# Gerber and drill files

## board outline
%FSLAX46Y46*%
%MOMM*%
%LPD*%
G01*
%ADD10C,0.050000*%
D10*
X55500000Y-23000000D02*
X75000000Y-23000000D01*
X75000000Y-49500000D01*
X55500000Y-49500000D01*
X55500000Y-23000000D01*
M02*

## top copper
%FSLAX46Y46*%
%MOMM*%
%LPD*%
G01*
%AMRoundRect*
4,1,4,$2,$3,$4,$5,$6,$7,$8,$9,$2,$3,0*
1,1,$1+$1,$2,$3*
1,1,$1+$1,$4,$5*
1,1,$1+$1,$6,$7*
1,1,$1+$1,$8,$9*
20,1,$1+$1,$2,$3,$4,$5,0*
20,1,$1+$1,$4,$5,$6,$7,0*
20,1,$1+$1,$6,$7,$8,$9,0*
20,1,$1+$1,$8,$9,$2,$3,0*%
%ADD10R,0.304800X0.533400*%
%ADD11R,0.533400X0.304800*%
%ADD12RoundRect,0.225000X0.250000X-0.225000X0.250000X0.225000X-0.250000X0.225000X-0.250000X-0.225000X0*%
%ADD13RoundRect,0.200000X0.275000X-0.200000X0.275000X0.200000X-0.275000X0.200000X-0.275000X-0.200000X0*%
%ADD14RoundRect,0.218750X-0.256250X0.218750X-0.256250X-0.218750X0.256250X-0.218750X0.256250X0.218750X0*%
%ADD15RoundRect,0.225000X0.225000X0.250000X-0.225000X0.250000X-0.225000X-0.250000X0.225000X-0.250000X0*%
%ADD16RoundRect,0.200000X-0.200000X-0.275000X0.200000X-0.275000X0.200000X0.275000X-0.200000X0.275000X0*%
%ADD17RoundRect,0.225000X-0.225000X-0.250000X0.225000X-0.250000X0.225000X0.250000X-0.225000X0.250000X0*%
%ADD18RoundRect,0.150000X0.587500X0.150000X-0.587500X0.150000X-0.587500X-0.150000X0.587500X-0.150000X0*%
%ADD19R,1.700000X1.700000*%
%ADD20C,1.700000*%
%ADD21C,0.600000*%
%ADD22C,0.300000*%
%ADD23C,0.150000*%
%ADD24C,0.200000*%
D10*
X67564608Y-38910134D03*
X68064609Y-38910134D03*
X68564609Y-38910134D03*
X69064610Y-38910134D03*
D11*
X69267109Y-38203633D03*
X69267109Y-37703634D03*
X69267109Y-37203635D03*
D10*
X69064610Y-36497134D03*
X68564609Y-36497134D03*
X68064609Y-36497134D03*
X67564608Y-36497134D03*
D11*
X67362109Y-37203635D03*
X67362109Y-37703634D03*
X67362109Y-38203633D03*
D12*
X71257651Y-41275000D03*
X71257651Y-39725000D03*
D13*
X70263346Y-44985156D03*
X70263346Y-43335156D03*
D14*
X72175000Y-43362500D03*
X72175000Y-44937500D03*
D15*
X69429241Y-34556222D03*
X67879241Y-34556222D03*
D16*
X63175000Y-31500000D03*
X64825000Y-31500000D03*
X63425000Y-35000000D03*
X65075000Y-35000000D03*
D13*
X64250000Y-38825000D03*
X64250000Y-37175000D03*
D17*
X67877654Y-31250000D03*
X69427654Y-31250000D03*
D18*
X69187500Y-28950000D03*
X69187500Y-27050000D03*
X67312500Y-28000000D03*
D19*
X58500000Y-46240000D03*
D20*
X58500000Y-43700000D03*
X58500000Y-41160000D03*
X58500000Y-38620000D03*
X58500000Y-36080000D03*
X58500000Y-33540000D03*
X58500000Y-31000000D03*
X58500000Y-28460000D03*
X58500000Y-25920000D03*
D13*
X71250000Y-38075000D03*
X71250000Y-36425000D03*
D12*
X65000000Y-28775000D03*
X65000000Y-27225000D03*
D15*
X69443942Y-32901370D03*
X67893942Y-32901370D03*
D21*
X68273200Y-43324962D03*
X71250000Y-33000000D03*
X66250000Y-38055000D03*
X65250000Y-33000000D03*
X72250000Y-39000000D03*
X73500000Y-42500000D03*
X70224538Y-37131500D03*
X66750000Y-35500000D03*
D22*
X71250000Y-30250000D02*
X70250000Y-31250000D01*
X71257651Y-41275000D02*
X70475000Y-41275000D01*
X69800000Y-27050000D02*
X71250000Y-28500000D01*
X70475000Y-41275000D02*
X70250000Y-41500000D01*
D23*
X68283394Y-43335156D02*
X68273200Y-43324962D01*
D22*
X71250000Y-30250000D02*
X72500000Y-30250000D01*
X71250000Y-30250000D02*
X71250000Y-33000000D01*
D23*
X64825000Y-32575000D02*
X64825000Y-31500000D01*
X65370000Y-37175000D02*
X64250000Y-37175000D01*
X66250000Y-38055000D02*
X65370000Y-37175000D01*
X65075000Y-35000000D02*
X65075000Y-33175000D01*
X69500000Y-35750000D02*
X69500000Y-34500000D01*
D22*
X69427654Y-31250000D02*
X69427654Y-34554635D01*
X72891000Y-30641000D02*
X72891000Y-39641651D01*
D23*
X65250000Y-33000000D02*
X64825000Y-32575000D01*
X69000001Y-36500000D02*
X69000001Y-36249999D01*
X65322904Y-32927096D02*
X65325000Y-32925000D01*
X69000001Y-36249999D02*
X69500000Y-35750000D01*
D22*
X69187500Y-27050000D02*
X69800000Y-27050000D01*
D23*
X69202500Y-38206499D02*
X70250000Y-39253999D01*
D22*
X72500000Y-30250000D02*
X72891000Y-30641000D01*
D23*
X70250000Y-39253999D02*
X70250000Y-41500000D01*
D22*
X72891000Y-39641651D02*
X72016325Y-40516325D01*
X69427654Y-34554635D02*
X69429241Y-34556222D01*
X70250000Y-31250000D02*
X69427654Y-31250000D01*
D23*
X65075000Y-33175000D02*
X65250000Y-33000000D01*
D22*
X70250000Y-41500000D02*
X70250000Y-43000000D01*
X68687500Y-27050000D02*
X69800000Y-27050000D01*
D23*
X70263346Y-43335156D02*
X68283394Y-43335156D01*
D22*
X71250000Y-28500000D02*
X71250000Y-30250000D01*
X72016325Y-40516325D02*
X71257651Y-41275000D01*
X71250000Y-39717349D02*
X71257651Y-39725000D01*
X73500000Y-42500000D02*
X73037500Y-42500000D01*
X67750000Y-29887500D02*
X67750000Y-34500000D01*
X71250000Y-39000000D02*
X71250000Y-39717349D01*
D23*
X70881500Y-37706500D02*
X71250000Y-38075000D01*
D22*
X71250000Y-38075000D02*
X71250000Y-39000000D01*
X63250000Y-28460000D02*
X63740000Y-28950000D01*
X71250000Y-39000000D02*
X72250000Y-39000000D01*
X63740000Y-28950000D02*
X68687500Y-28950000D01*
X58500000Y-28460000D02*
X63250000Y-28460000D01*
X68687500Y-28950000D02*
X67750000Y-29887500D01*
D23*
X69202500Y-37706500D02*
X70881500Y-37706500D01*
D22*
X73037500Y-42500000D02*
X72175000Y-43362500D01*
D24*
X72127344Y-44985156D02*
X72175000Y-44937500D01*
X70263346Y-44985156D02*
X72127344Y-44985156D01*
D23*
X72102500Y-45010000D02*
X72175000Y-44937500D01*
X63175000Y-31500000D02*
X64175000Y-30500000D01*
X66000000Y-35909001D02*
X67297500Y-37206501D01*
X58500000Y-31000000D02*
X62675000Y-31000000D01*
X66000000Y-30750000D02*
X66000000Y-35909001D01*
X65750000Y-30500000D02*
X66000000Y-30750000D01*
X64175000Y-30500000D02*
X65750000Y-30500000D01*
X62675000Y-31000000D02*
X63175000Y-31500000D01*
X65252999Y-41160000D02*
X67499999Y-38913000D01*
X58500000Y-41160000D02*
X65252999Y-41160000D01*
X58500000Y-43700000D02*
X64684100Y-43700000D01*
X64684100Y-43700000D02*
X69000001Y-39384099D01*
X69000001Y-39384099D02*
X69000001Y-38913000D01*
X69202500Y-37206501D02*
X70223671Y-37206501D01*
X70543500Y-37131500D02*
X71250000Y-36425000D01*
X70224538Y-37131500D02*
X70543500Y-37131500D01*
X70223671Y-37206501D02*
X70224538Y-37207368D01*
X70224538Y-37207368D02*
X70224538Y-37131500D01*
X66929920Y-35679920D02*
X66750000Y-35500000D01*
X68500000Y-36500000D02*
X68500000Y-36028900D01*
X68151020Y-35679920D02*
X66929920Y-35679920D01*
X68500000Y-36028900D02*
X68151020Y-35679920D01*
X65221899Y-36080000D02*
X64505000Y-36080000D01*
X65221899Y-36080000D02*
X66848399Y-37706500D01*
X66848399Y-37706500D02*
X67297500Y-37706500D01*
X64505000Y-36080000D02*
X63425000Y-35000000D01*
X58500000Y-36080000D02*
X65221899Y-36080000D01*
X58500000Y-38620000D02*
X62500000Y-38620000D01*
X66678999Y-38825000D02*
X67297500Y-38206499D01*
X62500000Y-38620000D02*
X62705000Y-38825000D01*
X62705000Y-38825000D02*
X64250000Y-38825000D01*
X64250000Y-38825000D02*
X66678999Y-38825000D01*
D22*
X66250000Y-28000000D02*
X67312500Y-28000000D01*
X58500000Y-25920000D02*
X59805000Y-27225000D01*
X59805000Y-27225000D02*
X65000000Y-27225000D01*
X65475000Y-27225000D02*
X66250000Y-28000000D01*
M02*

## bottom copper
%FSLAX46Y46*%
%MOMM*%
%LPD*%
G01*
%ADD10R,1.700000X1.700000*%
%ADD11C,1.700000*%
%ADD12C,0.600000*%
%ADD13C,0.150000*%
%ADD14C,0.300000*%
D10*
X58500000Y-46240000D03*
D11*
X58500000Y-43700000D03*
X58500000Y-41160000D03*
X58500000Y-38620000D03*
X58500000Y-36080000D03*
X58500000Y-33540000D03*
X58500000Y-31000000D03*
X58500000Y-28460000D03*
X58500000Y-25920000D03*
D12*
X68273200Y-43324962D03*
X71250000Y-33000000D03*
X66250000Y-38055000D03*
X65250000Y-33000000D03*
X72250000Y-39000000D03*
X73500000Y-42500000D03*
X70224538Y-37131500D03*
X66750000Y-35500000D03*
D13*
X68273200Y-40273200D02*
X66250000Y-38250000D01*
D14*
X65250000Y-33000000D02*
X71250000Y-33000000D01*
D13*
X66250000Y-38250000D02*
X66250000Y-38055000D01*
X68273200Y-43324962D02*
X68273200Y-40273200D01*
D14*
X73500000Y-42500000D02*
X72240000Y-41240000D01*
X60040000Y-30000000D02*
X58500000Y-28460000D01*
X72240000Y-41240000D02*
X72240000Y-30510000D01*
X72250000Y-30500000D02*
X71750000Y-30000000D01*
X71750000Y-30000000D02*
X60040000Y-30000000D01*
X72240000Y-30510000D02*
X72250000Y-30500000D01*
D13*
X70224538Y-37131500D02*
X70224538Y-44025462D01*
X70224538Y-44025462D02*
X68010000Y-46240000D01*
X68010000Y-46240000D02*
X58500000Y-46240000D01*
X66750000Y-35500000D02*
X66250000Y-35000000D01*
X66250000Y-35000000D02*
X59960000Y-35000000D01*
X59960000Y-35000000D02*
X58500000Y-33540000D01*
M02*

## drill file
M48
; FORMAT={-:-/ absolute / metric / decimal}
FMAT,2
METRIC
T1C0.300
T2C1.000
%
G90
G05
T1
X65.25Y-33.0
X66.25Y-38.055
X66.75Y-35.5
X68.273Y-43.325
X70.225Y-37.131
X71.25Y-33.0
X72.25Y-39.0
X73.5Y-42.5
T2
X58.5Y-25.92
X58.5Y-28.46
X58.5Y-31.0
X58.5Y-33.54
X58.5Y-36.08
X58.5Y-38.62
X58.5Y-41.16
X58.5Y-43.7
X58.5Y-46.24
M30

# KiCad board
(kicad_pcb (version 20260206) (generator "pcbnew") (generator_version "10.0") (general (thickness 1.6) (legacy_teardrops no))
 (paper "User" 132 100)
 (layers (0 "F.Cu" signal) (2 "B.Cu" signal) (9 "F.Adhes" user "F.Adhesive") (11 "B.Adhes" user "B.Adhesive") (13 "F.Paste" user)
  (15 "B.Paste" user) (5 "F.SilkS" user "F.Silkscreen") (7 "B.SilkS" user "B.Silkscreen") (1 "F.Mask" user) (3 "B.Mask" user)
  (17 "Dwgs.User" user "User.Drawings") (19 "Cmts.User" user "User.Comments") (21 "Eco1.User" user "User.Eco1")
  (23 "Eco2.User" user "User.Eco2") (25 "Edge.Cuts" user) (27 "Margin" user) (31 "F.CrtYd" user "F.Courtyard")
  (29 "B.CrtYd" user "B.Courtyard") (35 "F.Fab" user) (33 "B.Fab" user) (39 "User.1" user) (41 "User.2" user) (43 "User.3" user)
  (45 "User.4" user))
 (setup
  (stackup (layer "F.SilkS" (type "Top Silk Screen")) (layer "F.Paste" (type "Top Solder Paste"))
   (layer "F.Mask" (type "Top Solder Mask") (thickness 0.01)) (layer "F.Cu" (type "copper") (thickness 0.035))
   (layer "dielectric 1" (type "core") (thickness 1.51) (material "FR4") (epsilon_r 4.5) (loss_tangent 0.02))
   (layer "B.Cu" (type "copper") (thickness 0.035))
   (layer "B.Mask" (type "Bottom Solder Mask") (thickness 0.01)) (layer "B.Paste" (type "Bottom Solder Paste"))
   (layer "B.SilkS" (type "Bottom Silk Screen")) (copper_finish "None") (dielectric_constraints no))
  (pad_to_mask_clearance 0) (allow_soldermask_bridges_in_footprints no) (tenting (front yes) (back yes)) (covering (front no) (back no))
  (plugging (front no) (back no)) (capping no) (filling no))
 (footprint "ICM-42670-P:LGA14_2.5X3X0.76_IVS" (layer "F.Cu") (at 68.314609 37.703634 90)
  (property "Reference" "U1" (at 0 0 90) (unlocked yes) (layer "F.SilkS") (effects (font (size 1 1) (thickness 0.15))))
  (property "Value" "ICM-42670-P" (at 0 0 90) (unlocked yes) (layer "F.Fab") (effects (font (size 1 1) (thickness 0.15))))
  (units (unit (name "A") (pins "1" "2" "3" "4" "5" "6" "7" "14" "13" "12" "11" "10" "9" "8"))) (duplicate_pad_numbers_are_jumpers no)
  (pad "1" smd rect (at -1.2065 -0.750001 180) (size 0.3048 0.5334) (layers "F.Cu" "F.Mask" "F.Paste") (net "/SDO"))
  (pad "2" smd rect (at -1.2065 -0.25 180) (size 0.3048 0.5334) (layers "F.Cu" "F.Mask" "F.Paste") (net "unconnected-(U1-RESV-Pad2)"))
  (pad "3" smd rect (at -1.2065 0.25 180) (size 0.3048 0.5334) (layers "F.Cu" "F.Mask" "F.Paste") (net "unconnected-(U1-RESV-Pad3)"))
  (pad "4" smd rect (at -1.2065 0.750001 180) (size 0.3048 0.5334) (layers "F.Cu" "F.Mask" "F.Paste") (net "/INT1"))
  (pad "5" smd rect (at -0.499999 0.9525 90) (size 0.3048 0.5334) (layers "F.Cu" "F.Mask" "F.Paste") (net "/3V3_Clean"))
  (pad "6" smd rect (at 0 0.9525 90) (size 0.3048 0.5334) (layers "F.Cu" "F.Mask" "F.Paste") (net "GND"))
  (pad "7" smd rect (at 0.499999 0.9525 90) (size 0.3048 0.5334) (layers "F.Cu" "F.Mask" "F.Paste") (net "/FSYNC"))
  (pad "8" smd rect (at 1.2065 0.750001 180) (size 0.3048 0.5334) (layers "F.Cu" "F.Mask" "F.Paste") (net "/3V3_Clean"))
  (pad "9" smd rect (at 1.2065 0.25 180) (size 0.3048 0.5334) (layers "F.Cu" "F.Mask" "F.Paste") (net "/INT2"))
  (pad "10" smd rect (at 1.2065 -0.25 180) (size 0.3048 0.5334) (layers "F.Cu" "F.Mask" "F.Paste") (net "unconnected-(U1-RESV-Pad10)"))
  (pad "11" smd rect (at 1.2065 -0.750001 180) (size 0.3048 0.5334) (layers "F.Cu" "F.Mask" "F.Paste") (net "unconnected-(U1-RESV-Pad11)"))
  (pad "12" smd rect (at 0.499999 -0.9525 90) (size 0.3048 0.5334) (layers "F.Cu" "F.Mask" "F.Paste") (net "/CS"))
  (pad "13" smd rect (at 0 -0.9525 90) (size 0.3048 0.5334) (layers "F.Cu" "F.Mask" "F.Paste") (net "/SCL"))
  (pad "14" smd rect (at -0.499999 -0.9525 90) (size 0.3048 0.5334) (layers "F.Cu" "F.Mask" "F.Paste") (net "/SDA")))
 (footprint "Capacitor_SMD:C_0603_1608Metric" (layer "F.Cu") (at 71.257651 40.5 90)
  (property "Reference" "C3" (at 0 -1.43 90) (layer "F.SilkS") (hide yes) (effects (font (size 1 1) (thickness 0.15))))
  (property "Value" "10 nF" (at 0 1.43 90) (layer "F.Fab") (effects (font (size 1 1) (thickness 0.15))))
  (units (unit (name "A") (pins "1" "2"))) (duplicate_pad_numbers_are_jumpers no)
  (pad "1" smd roundrect (at -0.775 0 90) (size 0.9 0.95) (layers "F.Cu" "F.Mask" "F.Paste") (roundrect_rratio 0.25) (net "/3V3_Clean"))
  (pad "2" smd roundrect (at 0.775 0 90) (size 0.9 0.95) (layers "F.Cu" "F.Mask" "F.Paste") (roundrect_rratio 0.25) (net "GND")))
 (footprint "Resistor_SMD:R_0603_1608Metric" (layer "F.Cu") (at 70.263346 44.160156 90)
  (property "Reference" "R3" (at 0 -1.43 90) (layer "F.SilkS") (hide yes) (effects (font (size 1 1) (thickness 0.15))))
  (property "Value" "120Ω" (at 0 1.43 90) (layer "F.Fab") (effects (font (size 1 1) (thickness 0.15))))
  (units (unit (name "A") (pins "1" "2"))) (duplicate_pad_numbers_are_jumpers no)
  (pad "1" smd roundrect (at -0.825 0 90) (size 0.8 0.95) (layers "F.Cu" "F.Mask" "F.Paste") (roundrect_rratio 0.25) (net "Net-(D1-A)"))
  (pad "2" smd roundrect (at 0.825 0 90) (size 0.8 0.95) (layers "F.Cu" "F.Mask" "F.Paste") (roundrect_rratio 0.25) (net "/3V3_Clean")))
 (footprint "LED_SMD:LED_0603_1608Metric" (layer "F.Cu") (at 72.175 44.15 -90)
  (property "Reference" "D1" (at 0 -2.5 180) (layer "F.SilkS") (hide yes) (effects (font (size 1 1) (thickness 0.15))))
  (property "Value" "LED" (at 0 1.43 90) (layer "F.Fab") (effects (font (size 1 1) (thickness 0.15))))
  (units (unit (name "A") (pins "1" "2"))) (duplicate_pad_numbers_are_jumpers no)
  (pad "1" smd roundrect (at -0.7875 0 270) (size 0.875 0.95) (layers "F.Cu" "F.Mask" "F.Paste") (roundrect_rratio 0.25) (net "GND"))
  (pad "2" smd roundrect (at 0.7875 0 270) (size 0.875 0.95) (layers "F.Cu" "F.Mask" "F.Paste") (roundrect_rratio 0.25) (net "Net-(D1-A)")))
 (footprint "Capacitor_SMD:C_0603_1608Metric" (layer "F.Cu") (at 68.654241 34.556222 180)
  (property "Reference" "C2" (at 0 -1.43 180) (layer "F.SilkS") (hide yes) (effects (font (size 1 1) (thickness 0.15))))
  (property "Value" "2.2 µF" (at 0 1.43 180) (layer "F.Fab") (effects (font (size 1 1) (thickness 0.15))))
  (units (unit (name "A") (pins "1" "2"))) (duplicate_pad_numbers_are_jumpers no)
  (pad "1" smd roundrect (at -0.775 0 180) (size 0.9 0.95) (layers "F.Cu" "F.Mask" "F.Paste") (roundrect_rratio 0.25) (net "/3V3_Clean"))
  (pad "2" smd roundrect (at 0.775 0 180) (size 0.9 0.95) (layers "F.Cu" "F.Mask" "F.Paste") (roundrect_rratio 0.25) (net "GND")))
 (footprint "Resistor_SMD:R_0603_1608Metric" (layer "F.Cu") (at 64 31.5)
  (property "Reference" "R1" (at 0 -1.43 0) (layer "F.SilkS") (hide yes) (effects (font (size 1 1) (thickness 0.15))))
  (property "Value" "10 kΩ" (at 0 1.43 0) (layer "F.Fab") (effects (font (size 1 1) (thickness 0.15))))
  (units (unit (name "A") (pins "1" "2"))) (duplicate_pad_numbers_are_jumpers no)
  (pad "1" smd roundrect (at -0.825 0) (size 0.8 0.95) (layers "F.Cu" "F.Mask" "F.Paste") (roundrect_rratio 0.25) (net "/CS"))
  (pad "2" smd roundrect (at 0.825 0) (size 0.8 0.95) (layers "F.Cu" "F.Mask" "F.Paste") (roundrect_rratio 0.25) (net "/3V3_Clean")))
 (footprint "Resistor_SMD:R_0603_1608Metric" (layer "F.Cu") (at 64.25 35)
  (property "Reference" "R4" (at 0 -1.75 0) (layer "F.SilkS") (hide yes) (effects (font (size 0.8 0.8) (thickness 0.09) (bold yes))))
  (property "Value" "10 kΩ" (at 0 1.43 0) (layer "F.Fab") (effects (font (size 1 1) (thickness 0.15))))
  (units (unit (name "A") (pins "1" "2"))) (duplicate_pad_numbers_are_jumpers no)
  (pad "1" smd roundrect (at -0.825 0) (size 0.8 0.95) (layers "F.Cu" "F.Mask" "F.Paste") (roundrect_rratio 0.25) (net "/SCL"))
  (pad "2" smd roundrect (at 0.825 0) (size 0.8 0.95) (layers "F.Cu" "F.Mask" "F.Paste") (roundrect_rratio 0.25) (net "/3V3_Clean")))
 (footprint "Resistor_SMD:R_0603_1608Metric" (layer "F.Cu") (at 64.25 38 90)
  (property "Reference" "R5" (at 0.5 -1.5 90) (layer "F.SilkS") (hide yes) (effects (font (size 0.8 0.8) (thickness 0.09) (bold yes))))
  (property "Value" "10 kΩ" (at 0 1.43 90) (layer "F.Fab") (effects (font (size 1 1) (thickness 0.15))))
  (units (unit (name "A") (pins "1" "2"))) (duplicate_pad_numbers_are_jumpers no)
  (pad "1" smd roundrect (at -0.825 0 90) (size 0.8 0.95) (layers "F.Cu" "F.Mask" "F.Paste") (roundrect_rratio 0.25) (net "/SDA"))
  (pad "2" smd roundrect (at 0.825 0 90) (size 0.8 0.95) (layers "F.Cu" "F.Mask" "F.Paste") (roundrect_rratio 0.25) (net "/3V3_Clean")))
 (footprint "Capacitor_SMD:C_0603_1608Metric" (layer "F.Cu") (at 68.652654 31.25)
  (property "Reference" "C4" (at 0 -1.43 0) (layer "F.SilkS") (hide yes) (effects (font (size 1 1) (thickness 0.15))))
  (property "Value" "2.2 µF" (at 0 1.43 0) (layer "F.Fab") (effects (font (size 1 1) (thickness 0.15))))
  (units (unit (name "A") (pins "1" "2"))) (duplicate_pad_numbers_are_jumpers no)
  (pad "1" smd roundrect (at -0.775 0) (size 0.9 0.95) (layers "F.Cu" "F.Mask" "F.Paste") (roundrect_rratio 0.25) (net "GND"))
  (pad "2" smd roundrect (at 0.775 0) (size 0.9 0.95) (layers "F.Cu" "F.Mask" "F.Paste") (roundrect_rratio 0.25) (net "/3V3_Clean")))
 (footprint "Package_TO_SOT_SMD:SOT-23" (layer "F.Cu") (at 68.25 28 180)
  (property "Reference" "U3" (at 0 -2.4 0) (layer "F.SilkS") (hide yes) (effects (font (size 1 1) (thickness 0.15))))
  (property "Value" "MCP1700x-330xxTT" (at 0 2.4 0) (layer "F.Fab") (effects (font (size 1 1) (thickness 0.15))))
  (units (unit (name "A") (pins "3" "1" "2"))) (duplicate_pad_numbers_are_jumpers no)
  (pad "1" smd roundrect (at -0.9375 -0.95 180) (size 1.475 0.6) (layers "F.Cu" "F.Mask" "F.Paste") (roundrect_rratio 0.25) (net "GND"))
  (pad "2" smd roundrect (at -0.9375 0.95 180) (size 1.475 0.6) (layers "F.Cu" "F.Mask" "F.Paste") (roundrect_rratio 0.25)
   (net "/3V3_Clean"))
  (pad "3" smd roundrect (at 0.9375 0 180) (size 1.475 0.6) (layers "F.Cu" "F.Mask" "F.Paste") (roundrect_rratio 0.25)
   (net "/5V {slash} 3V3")))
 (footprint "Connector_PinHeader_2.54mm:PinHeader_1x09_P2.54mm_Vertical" (layer "F.Cu") (at 58.5 46.24 180)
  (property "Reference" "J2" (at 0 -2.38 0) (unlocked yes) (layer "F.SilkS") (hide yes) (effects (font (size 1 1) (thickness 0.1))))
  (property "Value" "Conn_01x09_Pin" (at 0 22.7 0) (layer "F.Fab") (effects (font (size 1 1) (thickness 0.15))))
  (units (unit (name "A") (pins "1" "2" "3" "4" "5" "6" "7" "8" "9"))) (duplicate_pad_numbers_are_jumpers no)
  (pad "1" thru_hole rect (at 0 0 180) (size 1.7 1.7) (drill 1) (layers "*.Cu" "*.Mask") (remove_unused_layers no) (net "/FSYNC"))
  (pad "2" thru_hole circle (at 0 2.54 180) (size 1.7 1.7) (drill 1) (layers "*.Cu" "*.Mask") (remove_unused_layers no) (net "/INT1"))
  (pad "3" thru_hole circle (at 0 5.08 180) (size 1.7 1.7) (drill 1) (layers "*.Cu" "*.Mask") (remove_unused_layers no) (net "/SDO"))
  (pad "4" thru_hole circle (at 0 7.62 180) (size 1.7 1.7) (drill 1) (layers "*.Cu" "*.Mask") (remove_unused_layers no) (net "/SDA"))
  (pad "5" thru_hole circle (at 0 10.16 180) (size 1.7 1.7) (drill 1) (layers "*.Cu" "*.Mask") (remove_unused_layers no) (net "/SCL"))
  (pad "6" thru_hole circle (at 0 12.7 180) (size 1.7 1.7) (drill 1) (layers "*.Cu" "*.Mask") (remove_unused_layers no) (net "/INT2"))
  (pad "7" thru_hole circle (at 0 15.24 180) (size 1.7 1.7) (drill 1) (layers "*.Cu" "*.Mask") (remove_unused_layers no) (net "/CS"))
  (pad "8" thru_hole circle (at 0 17.78 180) (size 1.7 1.7) (drill 1) (layers "*.Cu" "*.Mask") (remove_unused_layers no) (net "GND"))
  (pad "9" thru_hole circle (at 0 20.32 180) (size 1.7 1.7) (drill 1) (layers "*.Cu" "*.Mask") (remove_unused_layers no)
   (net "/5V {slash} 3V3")))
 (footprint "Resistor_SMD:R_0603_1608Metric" (layer "F.Cu") (at 71.25 37.25 90)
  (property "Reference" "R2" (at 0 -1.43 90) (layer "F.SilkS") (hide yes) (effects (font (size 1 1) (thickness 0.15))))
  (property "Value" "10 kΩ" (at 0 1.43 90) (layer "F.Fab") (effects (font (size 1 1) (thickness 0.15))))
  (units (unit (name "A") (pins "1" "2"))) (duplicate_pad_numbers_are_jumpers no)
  (pad "1" smd roundrect (at -0.825 0 90) (size 0.8 0.95) (layers "F.Cu" "F.Mask" "F.Paste") (roundrect_rratio 0.25) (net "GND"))
  (pad "2" smd roundrect (at 0.825 0 90) (size 0.8 0.95) (layers "F.Cu" "F.Mask" "F.Paste") (roundrect_rratio 0.25) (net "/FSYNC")))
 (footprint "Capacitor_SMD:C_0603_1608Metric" (layer "F.Cu") (at 65 28 90)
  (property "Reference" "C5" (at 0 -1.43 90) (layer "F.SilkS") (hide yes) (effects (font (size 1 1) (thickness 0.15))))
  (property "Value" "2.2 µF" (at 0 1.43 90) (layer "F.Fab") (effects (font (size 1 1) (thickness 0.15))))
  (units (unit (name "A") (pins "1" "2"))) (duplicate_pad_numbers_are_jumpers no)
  (pad "1" smd roundrect (at -0.775 0 90) (size 0.9 0.95) (layers "F.Cu" "F.Mask" "F.Paste") (roundrect_rratio 0.25) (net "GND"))
  (pad "2" smd roundrect (at 0.775 0 90) (size 0.9 0.95) (layers "F.Cu" "F.Mask" "F.Paste") (roundrect_rratio 0.25) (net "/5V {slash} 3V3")))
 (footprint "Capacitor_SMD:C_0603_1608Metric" (layer "F.Cu") (at 68.668942 32.90137 180)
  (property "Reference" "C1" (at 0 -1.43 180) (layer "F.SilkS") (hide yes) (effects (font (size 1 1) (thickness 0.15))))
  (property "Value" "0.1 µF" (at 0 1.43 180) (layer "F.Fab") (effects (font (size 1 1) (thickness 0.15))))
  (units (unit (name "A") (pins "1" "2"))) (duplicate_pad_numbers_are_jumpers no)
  (pad "1" smd roundrect (at -0.775 0 180) (size 0.9 0.95) (layers "F.Cu" "F.Mask" "F.Paste") (roundrect_rratio 0.25) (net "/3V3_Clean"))
  (pad "2" smd roundrect (at 0.775 0 180) (size 0.9 0.95) (layers "F.Cu" "F.Mask" "F.Paste") (roundrect_rratio 0.25) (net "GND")))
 (gr_rect (start 55.5 23) (end 75 49.5) (stroke (width 0.05) (type solid)) (fill no) (layer "Edge.Cuts"))
 (segment (start 71.25 30.25) (end 70.25 31.25) (width 0.3) (layer "F.Cu") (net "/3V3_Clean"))
 (segment (start 71.257651 41.275) (end 70.475 41.275) (width 0.3) (layer "F.Cu") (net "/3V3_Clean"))
 (segment (start 69.8 27.05) (end 71.25 28.5) (width 0.3) (layer "F.Cu") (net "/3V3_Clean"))
 (segment (start 70.475 41.275) (end 70.25 41.5) (width 0.3) (layer "F.Cu") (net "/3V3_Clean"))
 (segment (start 68.283394 43.335156) (end 68.2732 43.324962) (width 0.15) (layer "F.Cu") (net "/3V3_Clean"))
 (segment (start 71.25 30.25) (end 72.5 30.25) (width 0.3) (layer "F.Cu") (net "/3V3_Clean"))
 (segment (start 71.25 30.25) (end 71.25 33) (width 0.3) (layer "F.Cu") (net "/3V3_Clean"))
 (segment (start 64.825 32.575) (end 64.825 31.5) (width 0.15) (layer "F.Cu") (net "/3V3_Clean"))
 (segment (start 65.37 37.175) (end 64.25 37.175) (width 0.15) (layer "F.Cu") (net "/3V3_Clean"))
 (segment (start 66.25 38.055) (end 65.37 37.175) (width 0.15) (layer "F.Cu") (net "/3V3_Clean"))
 (segment (start 65.075 35) (end 65.075 33.175) (width 0.15) (layer "F.Cu") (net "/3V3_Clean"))
 (segment (start 69.5 35.75) (end 69.5 34.5) (width 0.15) (layer "F.Cu") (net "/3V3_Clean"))
 (segment (start 69.427654 31.25) (end 69.427654 34.554635) (width 0.3) (layer "F.Cu") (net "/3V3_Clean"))
 (segment (start 72.891 30.641) (end 72.891 39.641651) (width 0.3) (layer "F.Cu") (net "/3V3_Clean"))
 (segment (start 65.25 33) (end 64.825 32.575) (width 0.15) (layer "F.Cu") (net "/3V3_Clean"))
 (segment (start 69.000001 36.5) (end 69.000001 36.249999) (width 0.15) (layer "F.Cu") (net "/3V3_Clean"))
 (segment (start 65.322904 32.927096) (end 65.325 32.925) (width 0.15) (layer "F.Cu") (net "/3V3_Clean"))
 (segment (start 69.000001 36.249999) (end 69.5 35.75) (width 0.15) (layer "F.Cu") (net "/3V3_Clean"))
 (segment (start 69.1875 27.05) (end 69.8 27.05) (width 0.3) (layer "F.Cu") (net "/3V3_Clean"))
 (segment (start 69.2025 38.206499) (end 70.25 39.253999) (width 0.15) (layer "F.Cu") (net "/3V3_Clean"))
 (segment (start 72.5 30.25) (end 72.891 30.641) (width 0.3) (layer "F.Cu") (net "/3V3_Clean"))
 (segment (start 70.25 39.253999) (end 70.25 41.5) (width 0.15) (layer "F.Cu") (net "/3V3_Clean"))
 (segment (start 72.891 39.641651) (end 72.016325 40.516325) (width 0.3) (layer "F.Cu") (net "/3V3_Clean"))
 (segment (start 69.427654 34.554635) (end 69.429241 34.556222) (width 0.3) (layer "F.Cu") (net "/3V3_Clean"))
 (segment (start 70.25 31.25) (end 69.427654 31.25) (width 0.3) (layer "F.Cu") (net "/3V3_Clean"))
 (segment (start 65.075 33.175) (end 65.25 33) (width 0.15) (layer "F.Cu") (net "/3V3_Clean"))
 (segment (start 70.25 41.5) (end 70.25 43) (width 0.3) (layer "F.Cu") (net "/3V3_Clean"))
 (segment (start 68.6875 27.05) (end 69.8 27.05) (width 0.3) (layer "F.Cu") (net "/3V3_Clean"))
 (segment (start 70.263346 43.335156) (end 68.283394 43.335156) (width 0.15) (layer "F.Cu") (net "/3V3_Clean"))
 (segment (start 71.25 28.5) (end 71.25 30.25) (width 0.3) (layer "F.Cu") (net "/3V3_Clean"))
 (segment (start 72.016325 40.516325) (end 71.257651 41.275) (width 0.3) (layer "F.Cu") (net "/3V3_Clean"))
 (via (at 68.2732 43.324962) (size 0.6) (drill 0.3) (layers "F.Cu" "B.Cu") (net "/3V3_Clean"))
 (via (at 71.25 33) (size 0.6) (drill 0.3) (layers "F.Cu" "B.Cu") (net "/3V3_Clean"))
 (via (at 66.25 38.055) (size 0.6) (drill 0.3) (layers "F.Cu" "B.Cu") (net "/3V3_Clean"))
 (via (at 65.25 33) (size 0.6) (drill 0.3) (layers "F.Cu" "B.Cu") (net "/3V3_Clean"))
 (segment (start 68.2732 40.2732) (end 66.25 38.25) (width 0.15) (layer "B.Cu") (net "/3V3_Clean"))
 (segment (start 65.25 33) (end 71.25 33) (width 0.3) (layer "B.Cu") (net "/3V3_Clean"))
 (segment (start 66.25 38.25) (end 66.25 38.055) (width 0.15) (layer "B.Cu") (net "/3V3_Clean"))
 (segment (start 68.2732 43.324962) (end 68.2732 40.2732) (width 0.15) (layer "B.Cu") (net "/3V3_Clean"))
 (segment (start 71.25 39.717349) (end 71.257651 39.725) (width 0.3) (layer "F.Cu") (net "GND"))
 (segment (start 73.5 42.5) (end 73.0375 42.5) (width 0.3) (layer "F.Cu") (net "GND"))
 (segment (start 67.75 29.8875) (end 67.75 34.5) (width 0.3) (layer "F.Cu") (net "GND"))
 (segment (start 71.25 39) (end 71.25 39.717349) (width 0.3) (layer "F.Cu") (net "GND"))
 (segment (start 70.8815 37.7065) (end 71.25 38.075) (width 0.15) (layer "F.Cu") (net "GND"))
 (segment (start 71.25 38.075) (end 71.25 39) (width 0.3) (layer "F.Cu") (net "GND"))
 (segment (start 63.25 28.46) (end 63.74 28.95) (width 0.3) (layer "F.Cu") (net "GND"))
 (segment (start 71.25 39) (end 72.25 39) (width 0.3) (layer "F.Cu") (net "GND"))
 (segment (start 63.74 28.95) (end 68.6875 28.95) (width 0.3) (layer "F.Cu") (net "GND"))
 (segment (start 58.5 28.46) (end 63.25 28.46) (width 0.3) (layer "F.Cu") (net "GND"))
 (segment (start 68.6875 28.95) (end 67.75 29.8875) (width 0.3) (layer "F.Cu") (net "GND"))
 (segment (start 69.2025 37.7065) (end 70.8815 37.7065) (width 0.15) (layer "F.Cu") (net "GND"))
 (segment (start 73.0375 42.5) (end 72.175 43.3625) (width 0.3) (layer "F.Cu") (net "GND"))
 (via (at 72.25 39) (size 0.6) (drill 0.3) (layers "F.Cu" "B.Cu") (capping no) (covering (front no) (back no))
  (plugging (front no) (back no)) (filling no) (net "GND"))
 (via (at 73.5 42.5) (size 0.6) (drill 0.3) (layers "F.Cu" "B.Cu") (capping no) (covering (front no) (back no))
  (plugging (front no) (back no)) (filling no) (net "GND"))
 (segment (start 73.5 42.5) (end 72.24 41.24) (width 0.3) (layer "B.Cu") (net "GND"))
 (segment (start 60.04 30) (end 58.5 28.46) (width 0.3) (layer "B.Cu") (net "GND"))
 (segment (start 72.24 41.24) (end 72.24 30.51) (width 0.3) (layer "B.Cu") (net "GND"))
 (segment (start 72.25 30.5) (end 71.75 30) (width 0.3) (layer "B.Cu") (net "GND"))
 (segment (start 71.75 30) (end 60.04 30) (width 0.3) (layer "B.Cu") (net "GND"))
 (segment (start 72.24 30.51) (end 72.25 30.5) (width 0.3) (layer "B.Cu") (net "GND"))
 (segment (start 72.127344 44.985156) (end 72.175 44.9375) (width 0.2) (layer "F.Cu") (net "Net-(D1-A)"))
 (segment (start 70.263346 44.985156) (end 72.127344 44.985156) (width 0.2) (layer "F.Cu") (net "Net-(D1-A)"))
 (segment (start 72.1025 45.01) (end 72.175 44.9375) (width 0.15) (layer "F.Cu") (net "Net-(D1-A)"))
 (segment (start 63.175 31.5) (end 64.175 30.5) (width 0.15) (layer "F.Cu") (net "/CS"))
 (segment (start 66 35.909001) (end 67.2975 37.206501) (width 0.15) (layer "F.Cu") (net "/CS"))
 (segment (start 58.5 31) (end 62.675 31) (width 0.15) (layer "F.Cu") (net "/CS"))
 (segment (start 66 30.75) (end 66 35.909001) (width 0.15) (layer "F.Cu") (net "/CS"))
 (segment (start 65.75 30.5) (end 66 30.75) (width 0.15) (layer "F.Cu") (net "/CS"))
 (segment (start 64.175 30.5) (end 65.75 30.5) (width 0.15) (layer "F.Cu") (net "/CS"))
 (segment (start 62.675 31) (end 63.175 31.5) (width 0.15) (layer "F.Cu") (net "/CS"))
 (segment (start 65.252999 41.16) (end 67.499999 38.913) (width 0.15) (layer "F.Cu") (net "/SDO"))
 (segment (start 58.5 41.16) (end 65.252999 41.16) (width 0.15) (layer "F.Cu") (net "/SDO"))
 (segment (start 58.5 43.7) (end 64.6841 43.7) (width 0.15) (layer "F.Cu") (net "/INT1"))
 (segment (start 64.6841 43.7) (end 69.000001 39.384099) (width 0.15) (layer "F.Cu") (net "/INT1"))
 (segment (start 69.000001 39.384099) (end 69.000001 38.913) (width 0.15) (layer "F.Cu") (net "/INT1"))
 (segment (start 69.2025 37.206501) (end 70.223671 37.206501) (width 0.15) (layer "F.Cu") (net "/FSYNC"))
 (segment (start 70.5435 37.1315) (end 71.25 36.425) (width 0.15) (layer "F.Cu") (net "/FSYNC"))
 (segment (start 70.224538 37.1315) (end 70.5435 37.1315) (width 0.15) (layer "F.Cu") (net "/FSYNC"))
 (segment (start 70.223671 37.206501) (end 70.224538 37.207368) (width 0.15) (layer "F.Cu") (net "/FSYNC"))
 (segment (start 70.224538 37.207368) (end 70.224538 37.1315) (width 0.15) (layer "F.Cu") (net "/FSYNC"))
 (via (at 70.224538 37.1315) (size 0.6) (drill 0.3) (layers "F.Cu" "B.Cu") (capping no) (covering (front no) (back no))
  (plugging (front no) (back no)) (filling no) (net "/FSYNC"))
 (segment (start 70.224538 37.1315) (end 70.224538 44.025462) (width 0.15) (layer "B.Cu") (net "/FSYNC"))
 (segment (start 70.224538 44.025462) (end 68.01 46.24) (width 0.15) (layer "B.Cu") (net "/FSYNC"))
 (segment (start 68.01 46.24) (end 58.5 46.24) (width 0.15) (layer "B.Cu") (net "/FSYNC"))
 (segment (start 66.92992 35.67992) (end 66.75 35.5) (width 0.15) (layer "F.Cu") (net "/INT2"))
 (segment (start 68.5 36.5) (end 68.5 36.0289) (width 0.15) (layer "F.Cu") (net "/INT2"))
 (segment (start 68.15102 35.67992) (end 66.92992 35.67992) (width 0.15) (layer "F.Cu") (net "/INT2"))
 (segment (start 68.5 36.0289) (end 68.15102 35.67992) (width 0.15) (layer "F.Cu") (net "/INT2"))
 (via (at 66.75 35.5) (size 0.6) (drill 0.3) (layers "F.Cu" "B.Cu") (capping no) (covering (front no) (back no))
  (plugging (front no) (back no)) (filling no) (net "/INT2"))
 (segment (start 66.75 35.5) (end 66.25 35) (width 0.15) (layer "B.Cu") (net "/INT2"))
 (segment (start 66.25 35) (end 59.96 35) (width 0.15) (layer "B.Cu") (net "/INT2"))
 (segment (start 59.96 35) (end 58.5 33.54) (width 0.15) (layer "B.Cu") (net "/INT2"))
 (segment (start 65.221899 36.08) (end 64.505 36.08) (width 0.15) (layer "F.Cu") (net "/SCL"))
 (segment (start 65.221899 36.08) (end 66.848399 37.7065) (width 0.15) (layer "F.Cu") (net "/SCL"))
 (segment (start 66.848399 37.7065) (end 67.2975 37.7065) (width 0.15) (layer "F.Cu") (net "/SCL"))
 (segment (start 64.505 36.08) (end 63.425 35) (width 0.15) (layer "F.Cu") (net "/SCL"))
 (segment (start 58.5 36.08) (end 65.221899 36.08) (width 0.15) (layer "F.Cu") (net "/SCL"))
 (segment (start 58.5 38.62) (end 62.5 38.62) (width 0.15) (layer "F.Cu") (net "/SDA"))
 (segment (start 66.678999 38.825) (end 67.2975 38.206499) (width 0.15) (layer "F.Cu") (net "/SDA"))
 (segment (start 62.5 38.62) (end 62.705 38.825) (width 0.15) (layer "F.Cu") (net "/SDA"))
 (segment (start 62.705 38.825) (end 64.25 38.825) (width 0.15) (layer "F.Cu") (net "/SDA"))
 (segment (start 64.25 38.825) (end 66.678999 38.825) (width 0.15) (layer "F.Cu") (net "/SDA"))
 (segment (start 66.25 28) (end 67.3125 28) (width 0.3) (layer "F.Cu") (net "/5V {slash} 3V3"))
 (segment (start 58.5 25.92) (end 59.805 27.225) (width 0.3) (layer "F.Cu") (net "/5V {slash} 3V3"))
 (segment (start 59.805 27.225) (end 65 27.225) (width 0.3) (layer "F.Cu") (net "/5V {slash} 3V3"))
 (segment (start 65.475 27.225) (end 66.25 28) (width 0.3) (layer "F.Cu") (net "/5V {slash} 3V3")))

